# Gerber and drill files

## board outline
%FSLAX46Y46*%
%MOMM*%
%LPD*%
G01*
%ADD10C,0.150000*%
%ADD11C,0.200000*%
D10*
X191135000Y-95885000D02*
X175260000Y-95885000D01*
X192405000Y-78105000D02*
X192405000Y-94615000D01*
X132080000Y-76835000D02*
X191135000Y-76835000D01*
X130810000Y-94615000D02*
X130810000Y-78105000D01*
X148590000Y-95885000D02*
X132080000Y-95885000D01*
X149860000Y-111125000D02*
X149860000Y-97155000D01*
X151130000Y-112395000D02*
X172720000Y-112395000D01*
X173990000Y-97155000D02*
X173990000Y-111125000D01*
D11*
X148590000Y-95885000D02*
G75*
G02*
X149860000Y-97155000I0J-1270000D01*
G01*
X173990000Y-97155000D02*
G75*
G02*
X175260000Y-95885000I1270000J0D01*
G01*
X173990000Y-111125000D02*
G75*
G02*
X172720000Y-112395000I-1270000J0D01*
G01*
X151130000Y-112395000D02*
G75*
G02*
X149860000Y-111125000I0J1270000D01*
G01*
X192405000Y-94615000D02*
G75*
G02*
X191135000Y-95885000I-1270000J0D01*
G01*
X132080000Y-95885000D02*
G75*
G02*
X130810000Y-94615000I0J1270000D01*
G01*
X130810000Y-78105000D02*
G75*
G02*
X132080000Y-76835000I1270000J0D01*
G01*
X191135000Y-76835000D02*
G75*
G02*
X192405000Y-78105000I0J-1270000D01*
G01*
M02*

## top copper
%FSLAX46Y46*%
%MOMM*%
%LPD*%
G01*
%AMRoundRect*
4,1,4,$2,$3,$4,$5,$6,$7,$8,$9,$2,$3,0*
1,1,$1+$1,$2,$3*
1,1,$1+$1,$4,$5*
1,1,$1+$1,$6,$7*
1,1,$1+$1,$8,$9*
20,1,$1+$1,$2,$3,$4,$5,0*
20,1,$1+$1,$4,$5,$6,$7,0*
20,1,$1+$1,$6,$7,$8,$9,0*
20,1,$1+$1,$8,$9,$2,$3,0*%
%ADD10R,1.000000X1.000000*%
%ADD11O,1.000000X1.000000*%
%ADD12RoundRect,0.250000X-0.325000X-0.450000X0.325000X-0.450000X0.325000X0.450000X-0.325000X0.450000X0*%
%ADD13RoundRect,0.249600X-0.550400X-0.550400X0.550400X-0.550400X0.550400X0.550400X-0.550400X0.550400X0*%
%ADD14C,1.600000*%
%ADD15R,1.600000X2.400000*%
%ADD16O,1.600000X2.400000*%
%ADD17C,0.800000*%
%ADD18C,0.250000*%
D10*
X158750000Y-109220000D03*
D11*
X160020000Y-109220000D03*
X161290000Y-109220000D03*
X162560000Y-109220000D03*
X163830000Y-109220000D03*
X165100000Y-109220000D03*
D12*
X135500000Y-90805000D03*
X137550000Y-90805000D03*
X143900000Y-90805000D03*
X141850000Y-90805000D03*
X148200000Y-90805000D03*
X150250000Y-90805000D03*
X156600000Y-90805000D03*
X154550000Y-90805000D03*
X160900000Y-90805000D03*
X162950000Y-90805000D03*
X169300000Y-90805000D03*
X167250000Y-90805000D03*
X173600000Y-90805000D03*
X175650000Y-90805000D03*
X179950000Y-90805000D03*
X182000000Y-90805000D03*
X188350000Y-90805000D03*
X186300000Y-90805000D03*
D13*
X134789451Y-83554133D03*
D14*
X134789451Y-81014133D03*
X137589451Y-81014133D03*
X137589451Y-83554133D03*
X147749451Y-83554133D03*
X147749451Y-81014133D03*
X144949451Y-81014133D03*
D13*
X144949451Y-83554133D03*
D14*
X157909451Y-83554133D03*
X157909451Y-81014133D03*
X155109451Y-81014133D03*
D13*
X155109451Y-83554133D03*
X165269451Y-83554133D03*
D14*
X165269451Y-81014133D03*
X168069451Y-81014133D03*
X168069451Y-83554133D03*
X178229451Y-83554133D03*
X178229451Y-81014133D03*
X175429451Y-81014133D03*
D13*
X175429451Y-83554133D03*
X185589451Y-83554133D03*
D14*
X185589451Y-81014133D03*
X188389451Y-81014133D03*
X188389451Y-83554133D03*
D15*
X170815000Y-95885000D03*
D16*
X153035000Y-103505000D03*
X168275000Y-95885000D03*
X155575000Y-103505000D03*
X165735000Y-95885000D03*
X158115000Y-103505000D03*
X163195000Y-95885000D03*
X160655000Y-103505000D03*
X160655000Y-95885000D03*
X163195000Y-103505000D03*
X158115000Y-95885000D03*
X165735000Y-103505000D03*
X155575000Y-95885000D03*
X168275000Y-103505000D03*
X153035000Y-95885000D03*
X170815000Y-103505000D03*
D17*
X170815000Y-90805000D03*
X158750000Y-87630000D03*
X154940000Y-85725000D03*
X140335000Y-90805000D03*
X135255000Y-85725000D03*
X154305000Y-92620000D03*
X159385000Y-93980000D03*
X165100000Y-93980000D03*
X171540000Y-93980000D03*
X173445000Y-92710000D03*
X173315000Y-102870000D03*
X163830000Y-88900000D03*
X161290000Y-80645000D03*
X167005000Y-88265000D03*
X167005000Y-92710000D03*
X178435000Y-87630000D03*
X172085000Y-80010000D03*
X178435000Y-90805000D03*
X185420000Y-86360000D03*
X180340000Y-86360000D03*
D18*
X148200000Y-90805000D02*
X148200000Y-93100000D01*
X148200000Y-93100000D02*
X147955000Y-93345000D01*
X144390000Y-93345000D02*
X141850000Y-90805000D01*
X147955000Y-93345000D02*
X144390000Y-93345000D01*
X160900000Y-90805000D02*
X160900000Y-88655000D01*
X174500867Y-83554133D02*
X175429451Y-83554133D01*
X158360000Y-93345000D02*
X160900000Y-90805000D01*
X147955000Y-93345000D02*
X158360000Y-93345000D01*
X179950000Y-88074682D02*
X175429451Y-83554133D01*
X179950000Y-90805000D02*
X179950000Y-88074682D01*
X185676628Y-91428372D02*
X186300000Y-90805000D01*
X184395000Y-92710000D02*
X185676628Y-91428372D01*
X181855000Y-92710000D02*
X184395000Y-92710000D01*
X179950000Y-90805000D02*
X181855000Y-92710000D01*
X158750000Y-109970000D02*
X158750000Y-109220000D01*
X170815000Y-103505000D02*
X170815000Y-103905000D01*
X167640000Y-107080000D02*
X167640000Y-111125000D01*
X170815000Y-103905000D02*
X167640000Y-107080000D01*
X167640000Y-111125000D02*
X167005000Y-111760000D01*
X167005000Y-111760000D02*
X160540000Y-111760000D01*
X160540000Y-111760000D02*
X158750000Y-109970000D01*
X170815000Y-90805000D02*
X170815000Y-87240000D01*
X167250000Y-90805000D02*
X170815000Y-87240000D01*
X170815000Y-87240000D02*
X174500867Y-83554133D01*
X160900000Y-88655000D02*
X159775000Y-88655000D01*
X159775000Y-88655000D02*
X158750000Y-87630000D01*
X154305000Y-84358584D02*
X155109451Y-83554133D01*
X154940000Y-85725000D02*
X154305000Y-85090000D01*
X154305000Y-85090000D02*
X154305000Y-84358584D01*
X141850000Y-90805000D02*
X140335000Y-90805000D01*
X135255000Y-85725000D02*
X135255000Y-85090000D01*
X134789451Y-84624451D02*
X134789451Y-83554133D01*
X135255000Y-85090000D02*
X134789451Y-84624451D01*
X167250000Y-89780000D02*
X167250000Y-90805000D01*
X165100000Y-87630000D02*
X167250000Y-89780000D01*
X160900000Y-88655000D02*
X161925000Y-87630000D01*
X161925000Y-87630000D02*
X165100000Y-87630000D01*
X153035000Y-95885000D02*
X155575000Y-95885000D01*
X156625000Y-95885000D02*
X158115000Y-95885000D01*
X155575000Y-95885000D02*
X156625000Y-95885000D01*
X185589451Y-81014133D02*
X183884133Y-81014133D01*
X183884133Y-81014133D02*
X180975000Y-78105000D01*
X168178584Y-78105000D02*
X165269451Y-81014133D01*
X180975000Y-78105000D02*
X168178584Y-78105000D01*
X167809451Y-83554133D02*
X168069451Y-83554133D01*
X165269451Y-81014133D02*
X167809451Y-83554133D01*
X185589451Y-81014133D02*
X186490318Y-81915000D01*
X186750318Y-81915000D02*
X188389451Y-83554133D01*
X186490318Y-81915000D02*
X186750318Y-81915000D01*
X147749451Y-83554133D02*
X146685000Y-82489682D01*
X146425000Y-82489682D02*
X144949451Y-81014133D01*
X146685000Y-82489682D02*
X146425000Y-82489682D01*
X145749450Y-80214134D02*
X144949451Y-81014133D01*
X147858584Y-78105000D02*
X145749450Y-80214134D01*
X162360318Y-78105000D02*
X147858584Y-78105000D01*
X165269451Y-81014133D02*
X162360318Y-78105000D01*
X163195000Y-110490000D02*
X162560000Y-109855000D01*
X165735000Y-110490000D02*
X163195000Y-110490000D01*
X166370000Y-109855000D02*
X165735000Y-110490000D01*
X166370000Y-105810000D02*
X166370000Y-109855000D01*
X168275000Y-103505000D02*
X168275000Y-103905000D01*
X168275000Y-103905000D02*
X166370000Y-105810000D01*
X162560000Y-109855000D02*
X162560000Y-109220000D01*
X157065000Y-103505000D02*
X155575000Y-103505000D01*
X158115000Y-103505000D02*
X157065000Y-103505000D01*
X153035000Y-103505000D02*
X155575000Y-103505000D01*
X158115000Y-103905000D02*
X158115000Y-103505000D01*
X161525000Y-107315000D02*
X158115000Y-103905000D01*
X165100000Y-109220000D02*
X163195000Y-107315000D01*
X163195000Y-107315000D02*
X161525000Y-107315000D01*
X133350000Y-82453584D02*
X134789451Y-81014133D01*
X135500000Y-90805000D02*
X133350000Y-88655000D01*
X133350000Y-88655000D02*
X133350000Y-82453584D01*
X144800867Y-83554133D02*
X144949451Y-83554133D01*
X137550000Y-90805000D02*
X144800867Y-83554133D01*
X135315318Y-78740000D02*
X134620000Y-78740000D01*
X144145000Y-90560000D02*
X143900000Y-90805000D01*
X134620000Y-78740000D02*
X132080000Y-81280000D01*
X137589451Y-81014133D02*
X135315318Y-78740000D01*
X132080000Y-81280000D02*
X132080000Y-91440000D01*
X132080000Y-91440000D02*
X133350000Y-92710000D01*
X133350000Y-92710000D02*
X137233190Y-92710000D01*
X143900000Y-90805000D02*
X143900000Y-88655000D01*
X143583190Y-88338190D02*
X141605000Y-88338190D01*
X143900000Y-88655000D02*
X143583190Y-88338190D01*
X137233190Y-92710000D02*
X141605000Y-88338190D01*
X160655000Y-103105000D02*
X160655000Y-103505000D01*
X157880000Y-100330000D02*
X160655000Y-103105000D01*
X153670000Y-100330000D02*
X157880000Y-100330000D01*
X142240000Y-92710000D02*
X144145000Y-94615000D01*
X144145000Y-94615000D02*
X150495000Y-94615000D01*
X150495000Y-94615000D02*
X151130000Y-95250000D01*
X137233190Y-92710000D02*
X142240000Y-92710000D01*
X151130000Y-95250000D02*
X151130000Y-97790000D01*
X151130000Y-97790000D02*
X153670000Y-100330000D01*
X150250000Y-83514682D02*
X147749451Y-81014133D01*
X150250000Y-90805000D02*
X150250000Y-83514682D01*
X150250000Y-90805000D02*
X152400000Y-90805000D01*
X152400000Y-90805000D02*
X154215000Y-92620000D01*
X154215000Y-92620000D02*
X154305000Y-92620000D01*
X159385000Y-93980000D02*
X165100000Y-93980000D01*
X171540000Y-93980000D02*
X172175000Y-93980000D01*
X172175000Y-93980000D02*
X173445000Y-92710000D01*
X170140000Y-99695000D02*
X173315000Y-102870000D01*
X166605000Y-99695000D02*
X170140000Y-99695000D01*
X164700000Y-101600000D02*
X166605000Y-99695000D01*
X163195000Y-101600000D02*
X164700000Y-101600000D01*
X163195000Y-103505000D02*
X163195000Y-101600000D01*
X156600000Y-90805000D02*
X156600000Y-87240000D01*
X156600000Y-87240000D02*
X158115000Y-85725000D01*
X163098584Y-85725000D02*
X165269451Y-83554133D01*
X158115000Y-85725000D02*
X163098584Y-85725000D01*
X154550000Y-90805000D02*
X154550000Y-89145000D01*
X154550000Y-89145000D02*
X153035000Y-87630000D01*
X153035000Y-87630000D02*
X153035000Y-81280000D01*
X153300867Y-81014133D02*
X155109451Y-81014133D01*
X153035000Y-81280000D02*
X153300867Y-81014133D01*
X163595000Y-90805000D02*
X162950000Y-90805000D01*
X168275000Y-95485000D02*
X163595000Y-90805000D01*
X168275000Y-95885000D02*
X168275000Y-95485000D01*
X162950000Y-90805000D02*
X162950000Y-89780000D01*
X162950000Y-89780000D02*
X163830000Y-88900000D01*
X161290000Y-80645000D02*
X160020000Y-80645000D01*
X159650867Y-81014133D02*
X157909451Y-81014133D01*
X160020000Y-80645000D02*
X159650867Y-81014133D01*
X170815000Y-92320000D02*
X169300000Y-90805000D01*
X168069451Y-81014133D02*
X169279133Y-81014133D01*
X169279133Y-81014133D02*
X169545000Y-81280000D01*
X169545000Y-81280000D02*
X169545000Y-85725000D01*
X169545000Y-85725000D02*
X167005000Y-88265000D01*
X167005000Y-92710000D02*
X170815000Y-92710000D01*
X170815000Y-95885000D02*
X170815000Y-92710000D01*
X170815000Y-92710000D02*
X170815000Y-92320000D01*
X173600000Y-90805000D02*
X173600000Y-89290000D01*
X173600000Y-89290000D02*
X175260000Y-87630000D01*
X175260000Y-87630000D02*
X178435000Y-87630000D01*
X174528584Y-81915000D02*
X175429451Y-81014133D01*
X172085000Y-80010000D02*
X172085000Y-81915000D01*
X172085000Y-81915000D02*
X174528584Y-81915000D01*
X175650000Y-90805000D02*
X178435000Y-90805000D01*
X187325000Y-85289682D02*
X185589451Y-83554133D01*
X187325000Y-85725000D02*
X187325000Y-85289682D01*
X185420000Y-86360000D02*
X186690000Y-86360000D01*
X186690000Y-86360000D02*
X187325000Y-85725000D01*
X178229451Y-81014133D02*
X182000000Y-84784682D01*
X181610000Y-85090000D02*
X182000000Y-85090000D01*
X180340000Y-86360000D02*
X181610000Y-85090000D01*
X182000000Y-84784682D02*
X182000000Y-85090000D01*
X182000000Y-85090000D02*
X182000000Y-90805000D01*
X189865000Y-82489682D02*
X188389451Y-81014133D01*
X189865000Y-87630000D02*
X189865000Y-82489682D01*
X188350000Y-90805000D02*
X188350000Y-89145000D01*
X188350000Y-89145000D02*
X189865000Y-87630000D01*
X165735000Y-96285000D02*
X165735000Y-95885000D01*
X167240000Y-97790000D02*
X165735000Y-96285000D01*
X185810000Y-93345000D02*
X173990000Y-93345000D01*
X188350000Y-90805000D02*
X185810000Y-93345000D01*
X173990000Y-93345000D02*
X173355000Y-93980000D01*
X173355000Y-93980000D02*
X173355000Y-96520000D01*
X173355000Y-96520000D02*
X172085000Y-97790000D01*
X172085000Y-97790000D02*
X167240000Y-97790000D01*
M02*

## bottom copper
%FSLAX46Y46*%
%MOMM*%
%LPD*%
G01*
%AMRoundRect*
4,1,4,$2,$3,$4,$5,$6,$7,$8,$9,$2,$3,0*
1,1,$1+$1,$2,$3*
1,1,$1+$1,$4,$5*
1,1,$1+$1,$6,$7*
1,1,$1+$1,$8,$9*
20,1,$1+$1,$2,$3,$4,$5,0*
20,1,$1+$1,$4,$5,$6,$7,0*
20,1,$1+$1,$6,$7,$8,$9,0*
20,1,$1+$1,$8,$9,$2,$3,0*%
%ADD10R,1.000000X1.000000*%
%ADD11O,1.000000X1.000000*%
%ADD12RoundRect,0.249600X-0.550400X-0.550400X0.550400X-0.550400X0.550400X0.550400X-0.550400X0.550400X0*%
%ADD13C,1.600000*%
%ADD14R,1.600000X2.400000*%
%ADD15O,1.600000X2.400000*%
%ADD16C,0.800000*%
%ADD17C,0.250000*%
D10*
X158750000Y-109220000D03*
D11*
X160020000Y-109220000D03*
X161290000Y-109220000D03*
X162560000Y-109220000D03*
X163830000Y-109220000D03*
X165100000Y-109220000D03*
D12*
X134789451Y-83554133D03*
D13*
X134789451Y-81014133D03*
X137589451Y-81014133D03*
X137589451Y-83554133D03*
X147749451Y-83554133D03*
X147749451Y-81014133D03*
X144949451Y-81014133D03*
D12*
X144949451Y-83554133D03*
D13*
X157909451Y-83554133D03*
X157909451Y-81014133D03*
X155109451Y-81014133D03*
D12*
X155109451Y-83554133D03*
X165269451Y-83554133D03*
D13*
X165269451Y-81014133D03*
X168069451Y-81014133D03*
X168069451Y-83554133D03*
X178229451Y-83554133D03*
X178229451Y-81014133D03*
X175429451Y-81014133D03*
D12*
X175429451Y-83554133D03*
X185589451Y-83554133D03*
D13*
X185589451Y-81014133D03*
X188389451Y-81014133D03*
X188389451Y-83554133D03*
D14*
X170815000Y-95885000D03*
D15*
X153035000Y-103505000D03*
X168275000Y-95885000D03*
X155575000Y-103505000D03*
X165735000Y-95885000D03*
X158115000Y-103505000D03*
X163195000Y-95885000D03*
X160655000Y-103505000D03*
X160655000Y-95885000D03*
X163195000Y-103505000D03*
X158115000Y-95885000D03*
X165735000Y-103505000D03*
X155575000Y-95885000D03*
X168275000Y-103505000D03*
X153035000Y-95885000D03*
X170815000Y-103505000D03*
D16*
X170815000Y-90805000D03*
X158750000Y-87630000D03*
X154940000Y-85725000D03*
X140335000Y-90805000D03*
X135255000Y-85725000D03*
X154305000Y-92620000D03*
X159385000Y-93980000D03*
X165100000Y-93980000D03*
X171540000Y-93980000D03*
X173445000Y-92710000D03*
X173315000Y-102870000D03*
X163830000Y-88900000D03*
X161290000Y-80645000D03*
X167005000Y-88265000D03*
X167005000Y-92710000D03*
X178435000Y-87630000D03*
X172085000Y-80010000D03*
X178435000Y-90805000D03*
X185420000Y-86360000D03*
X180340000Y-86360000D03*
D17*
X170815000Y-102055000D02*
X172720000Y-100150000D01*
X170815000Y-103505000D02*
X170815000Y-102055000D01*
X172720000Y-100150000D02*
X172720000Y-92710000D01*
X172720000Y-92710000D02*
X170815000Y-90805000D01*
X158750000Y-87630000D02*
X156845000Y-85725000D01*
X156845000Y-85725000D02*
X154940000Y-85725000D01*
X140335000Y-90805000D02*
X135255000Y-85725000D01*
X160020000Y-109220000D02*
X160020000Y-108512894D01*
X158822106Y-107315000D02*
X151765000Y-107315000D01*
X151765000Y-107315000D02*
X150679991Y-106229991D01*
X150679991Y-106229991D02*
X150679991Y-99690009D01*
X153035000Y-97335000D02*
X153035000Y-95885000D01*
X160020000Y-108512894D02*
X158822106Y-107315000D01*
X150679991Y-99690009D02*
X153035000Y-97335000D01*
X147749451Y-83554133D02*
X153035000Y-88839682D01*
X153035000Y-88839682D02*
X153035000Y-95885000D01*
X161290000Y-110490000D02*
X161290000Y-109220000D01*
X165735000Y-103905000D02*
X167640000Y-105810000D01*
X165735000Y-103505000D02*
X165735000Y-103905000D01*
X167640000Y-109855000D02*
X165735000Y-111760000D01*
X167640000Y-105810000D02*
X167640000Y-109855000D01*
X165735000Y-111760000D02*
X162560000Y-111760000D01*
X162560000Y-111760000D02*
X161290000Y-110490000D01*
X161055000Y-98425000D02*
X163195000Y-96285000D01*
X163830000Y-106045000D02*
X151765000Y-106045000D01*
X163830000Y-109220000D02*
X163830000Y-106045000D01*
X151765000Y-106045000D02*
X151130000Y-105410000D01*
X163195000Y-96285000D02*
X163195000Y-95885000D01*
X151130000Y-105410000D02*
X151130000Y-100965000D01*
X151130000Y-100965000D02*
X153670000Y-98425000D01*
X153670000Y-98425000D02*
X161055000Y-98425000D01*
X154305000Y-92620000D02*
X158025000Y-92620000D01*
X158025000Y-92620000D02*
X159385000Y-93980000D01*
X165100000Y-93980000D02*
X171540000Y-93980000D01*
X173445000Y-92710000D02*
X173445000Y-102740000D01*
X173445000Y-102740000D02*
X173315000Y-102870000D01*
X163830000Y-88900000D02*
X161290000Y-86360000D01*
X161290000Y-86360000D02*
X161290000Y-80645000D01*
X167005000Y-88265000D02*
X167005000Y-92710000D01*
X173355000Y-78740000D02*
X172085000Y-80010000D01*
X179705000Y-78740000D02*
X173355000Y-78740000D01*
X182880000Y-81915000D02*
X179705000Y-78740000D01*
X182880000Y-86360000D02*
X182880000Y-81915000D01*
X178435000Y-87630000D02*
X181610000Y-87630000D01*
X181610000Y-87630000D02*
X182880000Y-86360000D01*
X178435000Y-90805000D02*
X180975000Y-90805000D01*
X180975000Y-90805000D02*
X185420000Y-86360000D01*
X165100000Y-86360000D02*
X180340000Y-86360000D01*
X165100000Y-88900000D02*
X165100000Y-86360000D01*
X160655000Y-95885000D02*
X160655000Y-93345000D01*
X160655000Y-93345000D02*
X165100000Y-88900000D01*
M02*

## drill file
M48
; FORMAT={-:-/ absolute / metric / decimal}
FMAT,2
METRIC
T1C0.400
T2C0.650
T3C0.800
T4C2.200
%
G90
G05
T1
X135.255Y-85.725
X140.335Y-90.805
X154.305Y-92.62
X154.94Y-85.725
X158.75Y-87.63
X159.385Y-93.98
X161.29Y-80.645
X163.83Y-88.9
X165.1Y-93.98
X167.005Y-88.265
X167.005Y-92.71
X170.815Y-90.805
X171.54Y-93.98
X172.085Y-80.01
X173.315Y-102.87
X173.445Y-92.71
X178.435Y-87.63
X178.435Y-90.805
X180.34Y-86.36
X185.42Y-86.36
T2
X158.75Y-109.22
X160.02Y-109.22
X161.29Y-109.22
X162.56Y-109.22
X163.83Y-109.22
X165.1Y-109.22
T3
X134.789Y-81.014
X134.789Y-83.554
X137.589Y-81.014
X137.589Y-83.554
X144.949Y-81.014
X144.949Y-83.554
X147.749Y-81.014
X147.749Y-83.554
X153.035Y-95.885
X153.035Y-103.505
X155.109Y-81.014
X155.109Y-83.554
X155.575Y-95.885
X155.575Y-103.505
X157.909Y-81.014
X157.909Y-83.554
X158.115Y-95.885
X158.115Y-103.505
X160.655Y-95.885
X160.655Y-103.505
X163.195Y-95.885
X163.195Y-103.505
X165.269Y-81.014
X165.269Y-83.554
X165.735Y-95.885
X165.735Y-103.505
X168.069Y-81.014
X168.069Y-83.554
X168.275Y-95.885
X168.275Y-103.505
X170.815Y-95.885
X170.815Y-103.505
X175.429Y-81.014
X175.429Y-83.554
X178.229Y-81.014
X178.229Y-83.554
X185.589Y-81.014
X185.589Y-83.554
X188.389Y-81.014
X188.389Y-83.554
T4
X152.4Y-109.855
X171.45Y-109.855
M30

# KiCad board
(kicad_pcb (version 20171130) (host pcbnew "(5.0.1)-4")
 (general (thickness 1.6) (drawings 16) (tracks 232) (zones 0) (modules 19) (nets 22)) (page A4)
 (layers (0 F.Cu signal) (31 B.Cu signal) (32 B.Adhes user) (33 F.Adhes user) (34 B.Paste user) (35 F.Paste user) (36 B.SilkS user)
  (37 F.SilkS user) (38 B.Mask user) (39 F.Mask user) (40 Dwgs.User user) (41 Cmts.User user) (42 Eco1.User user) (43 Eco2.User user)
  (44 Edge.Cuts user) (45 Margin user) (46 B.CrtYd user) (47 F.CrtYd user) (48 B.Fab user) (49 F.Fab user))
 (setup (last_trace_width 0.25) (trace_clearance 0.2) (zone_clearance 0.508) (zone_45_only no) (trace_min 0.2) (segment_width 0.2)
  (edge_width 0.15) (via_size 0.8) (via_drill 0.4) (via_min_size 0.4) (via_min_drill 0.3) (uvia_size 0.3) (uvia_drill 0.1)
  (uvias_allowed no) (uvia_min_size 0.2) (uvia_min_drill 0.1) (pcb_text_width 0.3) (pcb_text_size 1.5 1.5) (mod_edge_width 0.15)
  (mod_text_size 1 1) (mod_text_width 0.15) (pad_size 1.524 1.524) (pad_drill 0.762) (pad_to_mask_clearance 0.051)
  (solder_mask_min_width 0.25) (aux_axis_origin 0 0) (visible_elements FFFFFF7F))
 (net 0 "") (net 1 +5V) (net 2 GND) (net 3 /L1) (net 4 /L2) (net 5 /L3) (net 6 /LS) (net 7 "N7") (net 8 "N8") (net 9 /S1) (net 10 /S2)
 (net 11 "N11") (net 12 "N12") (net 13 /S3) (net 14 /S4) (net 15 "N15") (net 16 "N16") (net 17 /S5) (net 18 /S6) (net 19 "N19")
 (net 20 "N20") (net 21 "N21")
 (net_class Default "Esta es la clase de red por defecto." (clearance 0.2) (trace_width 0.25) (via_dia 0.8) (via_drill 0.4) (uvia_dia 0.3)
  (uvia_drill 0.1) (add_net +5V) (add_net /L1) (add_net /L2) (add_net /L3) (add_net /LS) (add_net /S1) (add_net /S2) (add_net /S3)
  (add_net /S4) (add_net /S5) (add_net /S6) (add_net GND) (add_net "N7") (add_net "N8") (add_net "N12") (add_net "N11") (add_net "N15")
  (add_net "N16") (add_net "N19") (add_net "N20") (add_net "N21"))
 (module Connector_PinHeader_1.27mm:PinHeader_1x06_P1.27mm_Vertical (layer F.Cu) (at 158.75 109.22 90)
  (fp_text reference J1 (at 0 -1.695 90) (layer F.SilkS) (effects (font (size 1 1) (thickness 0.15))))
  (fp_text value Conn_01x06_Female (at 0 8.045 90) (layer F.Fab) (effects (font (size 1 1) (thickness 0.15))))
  (pad 1 thru_hole rect (at 0 0 90) (size 1 1) (drill 0.65) (layers *.Cu *.Mask) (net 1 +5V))
  (pad 2 thru_hole oval (at 0 1.27 90) (size 1 1) (drill 0.65) (layers *.Cu *.Mask) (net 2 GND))
  (pad 3 thru_hole oval (at 0 2.54 90) (size 1 1) (drill 0.65) (layers *.Cu *.Mask) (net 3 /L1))
  (pad 4 thru_hole oval (at 0 3.81 90) (size 1 1) (drill 0.65) (layers *.Cu *.Mask) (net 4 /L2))
  (pad 5 thru_hole oval (at 0 5.08 90) (size 1 1) (drill 0.65) (layers *.Cu *.Mask) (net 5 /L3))
  (pad 6 thru_hole oval (at 0 6.35 90) (size 1 1) (drill 0.65) (layers *.Cu *.Mask) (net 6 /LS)))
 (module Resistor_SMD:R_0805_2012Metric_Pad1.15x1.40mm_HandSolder (layer F.Cu) (at 136.525 90.805)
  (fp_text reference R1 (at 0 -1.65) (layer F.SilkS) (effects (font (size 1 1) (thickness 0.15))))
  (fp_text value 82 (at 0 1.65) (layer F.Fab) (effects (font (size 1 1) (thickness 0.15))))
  (pad 1 smd roundrect (at -1.025 0) (size 1.15 1.4) (layers F.Cu F.Paste F.Mask) (roundrect_rratio 0.217391) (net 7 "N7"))
  (pad 2 smd roundrect (at 1.025 0) (size 1.15 1.4) (layers F.Cu F.Paste F.Mask) (roundrect_rratio 0.217391) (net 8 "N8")))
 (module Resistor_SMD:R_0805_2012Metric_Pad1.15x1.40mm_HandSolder (layer F.Cu) (at 142.875 90.805)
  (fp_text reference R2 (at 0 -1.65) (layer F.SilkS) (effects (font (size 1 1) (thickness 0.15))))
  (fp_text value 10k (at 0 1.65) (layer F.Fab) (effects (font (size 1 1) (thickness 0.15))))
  (pad 2 smd roundrect (at 1.025 0) (size 1.15 1.4) (layers F.Cu F.Paste F.Mask) (roundrect_rratio 0.217391) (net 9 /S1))
  (pad 1 smd roundrect (at -1.025 0) (size 1.15 1.4) (layers F.Cu F.Paste F.Mask) (roundrect_rratio 0.217391) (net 1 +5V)))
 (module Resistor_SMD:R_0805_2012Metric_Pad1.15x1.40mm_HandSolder (layer F.Cu) (at 149.225 90.805)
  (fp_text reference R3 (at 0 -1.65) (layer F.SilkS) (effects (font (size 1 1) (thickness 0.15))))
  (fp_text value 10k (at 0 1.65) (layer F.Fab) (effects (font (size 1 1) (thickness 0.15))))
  (pad 1 smd roundrect (at -1.025 0) (size 1.15 1.4) (layers F.Cu F.Paste F.Mask) (roundrect_rratio 0.217391) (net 1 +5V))
  (pad 2 smd roundrect (at 1.025 0) (size 1.15 1.4) (layers F.Cu F.Paste F.Mask) (roundrect_rratio 0.217391) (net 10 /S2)))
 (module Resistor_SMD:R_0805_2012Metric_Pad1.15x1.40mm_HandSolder (layer F.Cu) (at 155.575 90.805)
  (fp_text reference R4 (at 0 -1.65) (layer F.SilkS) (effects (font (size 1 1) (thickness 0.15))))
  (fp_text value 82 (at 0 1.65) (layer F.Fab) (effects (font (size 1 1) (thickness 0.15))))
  (pad 2 smd roundrect (at 1.025 0) (size 1.15 1.4) (layers F.Cu F.Paste F.Mask) (roundrect_rratio 0.217391) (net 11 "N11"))
  (pad 1 smd roundrect (at -1.025 0) (size 1.15 1.4) (layers F.Cu F.Paste F.Mask) (roundrect_rratio 0.217391) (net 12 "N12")))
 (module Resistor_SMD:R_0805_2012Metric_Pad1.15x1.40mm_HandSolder (layer F.Cu) (at 161.925 90.805)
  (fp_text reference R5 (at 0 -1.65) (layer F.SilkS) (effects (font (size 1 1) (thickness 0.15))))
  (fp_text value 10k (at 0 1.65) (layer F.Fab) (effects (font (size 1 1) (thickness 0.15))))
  (pad 1 smd roundrect (at -1.025 0) (size 1.15 1.4) (layers F.Cu F.Paste F.Mask) (roundrect_rratio 0.217391) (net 1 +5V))
  (pad 2 smd roundrect (at 1.025 0) (size 1.15 1.4) (layers F.Cu F.Paste F.Mask) (roundrect_rratio 0.217391) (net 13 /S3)))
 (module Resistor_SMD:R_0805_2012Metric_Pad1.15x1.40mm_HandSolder (layer F.Cu) (at 168.275 90.805)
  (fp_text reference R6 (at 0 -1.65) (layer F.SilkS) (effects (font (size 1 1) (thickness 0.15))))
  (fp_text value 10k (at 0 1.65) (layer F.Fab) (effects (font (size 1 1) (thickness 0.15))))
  (pad 2 smd roundrect (at 1.025 0) (size 1.15 1.4) (layers F.Cu F.Paste F.Mask) (roundrect_rratio 0.217391) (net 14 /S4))
  (pad 1 smd roundrect (at -1.025 0) (size 1.15 1.4) (layers F.Cu F.Paste F.Mask) (roundrect_rratio 0.217391) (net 1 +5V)))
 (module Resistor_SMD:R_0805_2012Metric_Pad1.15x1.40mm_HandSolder (layer F.Cu) (at 174.625 90.805)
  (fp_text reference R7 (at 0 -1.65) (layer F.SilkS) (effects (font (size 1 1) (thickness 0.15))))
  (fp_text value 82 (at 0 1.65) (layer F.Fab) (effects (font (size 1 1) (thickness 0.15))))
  (pad 1 smd roundrect (at -1.025 0) (size 1.15 1.4) (layers F.Cu F.Paste F.Mask) (roundrect_rratio 0.217391) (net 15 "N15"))
  (pad 2 smd roundrect (at 1.025 0) (size 1.15 1.4) (layers F.Cu F.Paste F.Mask) (roundrect_rratio 0.217391) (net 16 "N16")))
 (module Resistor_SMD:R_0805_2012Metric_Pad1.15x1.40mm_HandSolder (layer F.Cu) (at 180.975 90.805)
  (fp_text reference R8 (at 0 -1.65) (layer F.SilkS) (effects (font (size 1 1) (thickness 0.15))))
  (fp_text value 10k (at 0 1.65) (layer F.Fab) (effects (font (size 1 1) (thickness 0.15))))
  (pad 1 smd roundrect (at -1.025 0) (size 1.15 1.4) (layers F.Cu F.Paste F.Mask) (roundrect_rratio 0.217391) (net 1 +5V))
  (pad 2 smd roundrect (at 1.025 0) (size 1.15 1.4) (layers F.Cu F.Paste F.Mask) (roundrect_rratio 0.217391) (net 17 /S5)))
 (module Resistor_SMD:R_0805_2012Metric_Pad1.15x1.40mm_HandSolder (layer F.Cu) (at 187.325 90.805)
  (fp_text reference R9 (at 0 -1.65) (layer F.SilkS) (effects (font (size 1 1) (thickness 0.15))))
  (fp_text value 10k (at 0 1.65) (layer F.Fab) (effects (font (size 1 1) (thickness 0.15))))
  (pad 2 smd roundrect (at 1.025 0) (size 1.15 1.4) (layers F.Cu F.Paste F.Mask) (roundrect_rratio 0.217391) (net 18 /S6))
  (pad 1 smd roundrect (at -1.025 0) (size 1.15 1.4) (layers F.Cu F.Paste F.Mask) (roundrect_rratio 0.217391) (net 1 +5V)))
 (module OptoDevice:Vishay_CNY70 (layer B.Cu) (at 134.789451 83.554133)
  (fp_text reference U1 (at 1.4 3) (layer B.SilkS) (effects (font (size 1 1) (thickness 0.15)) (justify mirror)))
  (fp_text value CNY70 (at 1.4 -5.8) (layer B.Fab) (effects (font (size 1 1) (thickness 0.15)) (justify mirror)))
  (pad 1 thru_hole roundrect (at 0 0) (size 1.6 1.6) (drill 0.8) (layers *.Cu *.Mask) (roundrect_rratio 0.156) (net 1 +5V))
  (pad 2 thru_hole circle (at 0 -2.54) (size 1.6 1.6) (drill 0.8) (layers *.Cu *.Mask) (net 7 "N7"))
  (pad 3 thru_hole circle (at 2.8 -2.54) (size 1.6 1.6) (drill 0.8) (layers *.Cu *.Mask) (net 9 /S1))
  (pad 4 thru_hole circle (at 2.8 0) (size 1.6 1.6) (drill 0.8) (layers *.Cu *.Mask) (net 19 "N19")))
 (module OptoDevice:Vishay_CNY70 (layer B.Cu) (at 144.949451 83.554133)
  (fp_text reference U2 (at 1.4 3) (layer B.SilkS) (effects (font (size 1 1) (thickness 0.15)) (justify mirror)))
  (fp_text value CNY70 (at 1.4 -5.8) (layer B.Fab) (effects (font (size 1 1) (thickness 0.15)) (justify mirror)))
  (pad 4 thru_hole circle (at 2.8 0) (size 1.6 1.6) (drill 0.8) (layers *.Cu *.Mask) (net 2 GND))
  (pad 3 thru_hole circle (at 2.8 -2.54) (size 1.6 1.6) (drill 0.8) (layers *.Cu *.Mask) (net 10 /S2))
  (pad 2 thru_hole circle (at 0 -2.54) (size 1.6 1.6) (drill 0.8) (layers *.Cu *.Mask) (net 2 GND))
  (pad 1 thru_hole roundrect (at 0 0) (size 1.6 1.6) (drill 0.8) (layers *.Cu *.Mask) (roundrect_rratio 0.156) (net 8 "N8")))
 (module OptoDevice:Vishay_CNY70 (layer B.Cu) (at 155.109451 83.554133)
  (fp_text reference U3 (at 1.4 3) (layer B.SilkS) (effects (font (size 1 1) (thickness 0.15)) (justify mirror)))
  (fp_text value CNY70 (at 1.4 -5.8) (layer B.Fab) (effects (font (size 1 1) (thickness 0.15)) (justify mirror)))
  (pad 4 thru_hole circle (at 2.8 0) (size 1.6 1.6) (drill 0.8) (layers *.Cu *.Mask) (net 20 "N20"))
  (pad 3 thru_hole circle (at 2.8 -2.54) (size 1.6 1.6) (drill 0.8) (layers *.Cu *.Mask) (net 13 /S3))
  (pad 2 thru_hole circle (at 0 -2.54) (size 1.6 1.6) (drill 0.8) (layers *.Cu *.Mask) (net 12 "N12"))
  (pad 1 thru_hole roundrect (at 0 0) (size 1.6 1.6) (drill 0.8) (layers *.Cu *.Mask) (roundrect_rratio 0.156) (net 1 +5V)))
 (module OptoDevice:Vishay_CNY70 (layer B.Cu) (at 165.269451 83.554133)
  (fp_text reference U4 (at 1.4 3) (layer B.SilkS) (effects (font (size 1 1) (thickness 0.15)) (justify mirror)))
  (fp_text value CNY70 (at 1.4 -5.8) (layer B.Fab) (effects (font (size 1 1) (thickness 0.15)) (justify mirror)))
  (pad 1 thru_hole roundrect (at 0 0) (size 1.6 1.6) (drill 0.8) (layers *.Cu *.Mask) (roundrect_rratio 0.156) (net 11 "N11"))
  (pad 2 thru_hole circle (at 0 -2.54) (size 1.6 1.6) (drill 0.8) (layers *.Cu *.Mask) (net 2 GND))
  (pad 3 thru_hole circle (at 2.8 -2.54) (size 1.6 1.6) (drill 0.8) (layers *.Cu *.Mask) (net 14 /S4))
  (pad 4 thru_hole circle (at 2.8 0) (size 1.6 1.6) (drill 0.8) (layers *.Cu *.Mask) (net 2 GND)))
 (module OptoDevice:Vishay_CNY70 (layer B.Cu) (at 175.429451 83.554133)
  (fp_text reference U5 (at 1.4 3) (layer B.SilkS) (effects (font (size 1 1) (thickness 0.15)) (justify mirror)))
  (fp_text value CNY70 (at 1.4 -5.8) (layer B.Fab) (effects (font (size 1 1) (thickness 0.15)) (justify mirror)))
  (pad 4 thru_hole circle (at 2.8 0) (size 1.6 1.6) (drill 0.8) (layers *.Cu *.Mask) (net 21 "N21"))
  (pad 3 thru_hole circle (at 2.8 -2.54) (size 1.6 1.6) (drill 0.8) (layers *.Cu *.Mask) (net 17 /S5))
  (pad 2 thru_hole circle (at 0 -2.54) (size 1.6 1.6) (drill 0.8) (layers *.Cu *.Mask) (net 15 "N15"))
  (pad 1 thru_hole roundrect (at 0 0) (size 1.6 1.6) (drill 0.8) (layers *.Cu *.Mask) (roundrect_rratio 0.156) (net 1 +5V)))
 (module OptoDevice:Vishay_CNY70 (layer B.Cu) (at 185.589451 83.554133)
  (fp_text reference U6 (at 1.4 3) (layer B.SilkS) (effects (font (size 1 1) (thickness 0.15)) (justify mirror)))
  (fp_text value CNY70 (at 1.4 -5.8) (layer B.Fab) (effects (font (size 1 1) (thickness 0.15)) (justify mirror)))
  (pad 1 thru_hole roundrect (at 0 0) (size 1.6 1.6) (drill 0.8) (layers *.Cu *.Mask) (roundrect_rratio 0.156) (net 16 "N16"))
  (pad 2 thru_hole circle (at 0 -2.54) (size 1.6 1.6) (drill 0.8) (layers *.Cu *.Mask) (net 2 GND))
  (pad 3 thru_hole circle (at 2.8 -2.54) (size 1.6 1.6) (drill 0.8) (layers *.Cu *.Mask) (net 18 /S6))
  (pad 4 thru_hole circle (at 2.8 0) (size 1.6 1.6) (drill 0.8) (layers *.Cu *.Mask) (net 2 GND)))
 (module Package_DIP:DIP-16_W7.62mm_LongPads (layer F.Cu) (at 170.815 95.885 270)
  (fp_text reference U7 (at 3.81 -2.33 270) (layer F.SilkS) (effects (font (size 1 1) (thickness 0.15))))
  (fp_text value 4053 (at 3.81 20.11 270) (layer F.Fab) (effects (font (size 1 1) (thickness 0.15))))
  (pad 1 thru_hole rect (at 0 0 270) (size 2.4 1.6) (drill 0.8) (layers *.Cu *.Mask) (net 14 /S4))
  (pad 9 thru_hole oval (at 7.62 17.78 270) (size 2.4 1.6) (drill 0.8) (layers *.Cu *.Mask) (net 6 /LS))
  (pad 2 thru_hole oval (at 0 2.54 270) (size 2.4 1.6) (drill 0.8) (layers *.Cu *.Mask) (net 13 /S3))
  (pad 10 thru_hole oval (at 7.62 15.24 270) (size 2.4 1.6) (drill 0.8) (layers *.Cu *.Mask) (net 6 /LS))
  (pad 3 thru_hole oval (at 0 5.08 270) (size 2.4 1.6) (drill 0.8) (layers *.Cu *.Mask) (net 18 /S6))
  (pad 11 thru_hole oval (at 7.62 12.7 270) (size 2.4 1.6) (drill 0.8) (layers *.Cu *.Mask) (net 6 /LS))
  (pad 4 thru_hole oval (at 0 7.62 270) (size 2.4 1.6) (drill 0.8) (layers *.Cu *.Mask) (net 5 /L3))
  (pad 12 thru_hole oval (at 7.62 10.16 270) (size 2.4 1.6) (drill 0.8) (layers *.Cu *.Mask) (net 9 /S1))
  (pad 5 thru_hole oval (at 0 10.16 270) (size 2.4 1.6) (drill 0.8) (layers *.Cu *.Mask) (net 17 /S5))
  (pad 13 thru_hole oval (at 7.62 7.62 270) (size 2.4 1.6) (drill 0.8) (layers *.Cu *.Mask) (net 10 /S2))
  (pad 6 thru_hole oval (at 0 12.7 270) (size 2.4 1.6) (drill 0.8) (layers *.Cu *.Mask) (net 2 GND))
  (pad 14 thru_hole oval (at 7.62 5.08 270) (size 2.4 1.6) (drill 0.8) (layers *.Cu *.Mask) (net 3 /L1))
  (pad 7 thru_hole oval (at 0 15.24 270) (size 2.4 1.6) (drill 0.8) (layers *.Cu *.Mask) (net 2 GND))
  (pad 15 thru_hole oval (at 7.62 2.54 270) (size 2.4 1.6) (drill 0.8) (layers *.Cu *.Mask) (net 4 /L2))
  (pad 8 thru_hole oval (at 0 17.78 270) (size 2.4 1.6) (drill 0.8) (layers *.Cu *.Mask) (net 2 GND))
  (pad 16 thru_hole oval (at 7.62 0 270) (size 2.4 1.6) (drill 0.8) (layers *.Cu *.Mask) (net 1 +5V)))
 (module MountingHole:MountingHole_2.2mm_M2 (layer F.Cu) (at 152.4 109.855)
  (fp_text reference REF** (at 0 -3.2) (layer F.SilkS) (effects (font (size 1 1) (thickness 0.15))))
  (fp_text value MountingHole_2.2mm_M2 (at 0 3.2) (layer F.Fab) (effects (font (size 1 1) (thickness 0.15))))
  (pad 1 np_thru_hole circle (at 0 0) (size 2.2 2.2) (drill 2.2) (layers *.Cu *.Mask)))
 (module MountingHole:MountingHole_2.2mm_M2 (layer F.Cu) (at 171.45 109.855)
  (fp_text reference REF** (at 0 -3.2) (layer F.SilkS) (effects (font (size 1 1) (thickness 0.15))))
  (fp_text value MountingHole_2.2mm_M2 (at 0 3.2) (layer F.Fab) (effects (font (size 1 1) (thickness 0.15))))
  (pad 1 np_thru_hole circle (at 0 0) (size 2.2 2.2) (drill 2.2) (layers *.Cu *.Mask)))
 (gr_line (start 191.135 95.885) (end 175.26 95.885) (layer Edge.Cuts) (width 0.15))
 (gr_line (start 192.405 78.105) (end 192.405 94.615) (layer Edge.Cuts) (width 0.15))
 (gr_line (start 132.08 76.835) (end 191.135 76.835) (layer Edge.Cuts) (width 0.15))
 (gr_line (start 130.81 94.615) (end 130.81 78.105) (layer Edge.Cuts) (width 0.15))
 (gr_line (start 148.59 95.885) (end 132.08 95.885) (layer Edge.Cuts) (width 0.15))
 (gr_line (start 149.86 111.125) (end 149.86 97.155) (layer Edge.Cuts) (width 0.15))
 (gr_line (start 151.13 112.395) (end 172.72 112.395) (layer Edge.Cuts) (width 0.15))
 (gr_line (start 173.99 97.155) (end 173.99 111.125) (layer Edge.Cuts) (width 0.15))
 (gr_arc (start 148.59 97.155) (end 149.86 97.155) (angle -90) (layer Edge.Cuts) (width 0.2))
 (gr_arc (start 175.26 97.155) (end 175.26 95.885) (angle -90) (layer Edge.Cuts) (width 0.2))
 (gr_arc (start 172.72 111.125) (end 172.72 112.395) (angle -90) (layer Edge.Cuts) (width 0.2))
 (gr_arc (start 151.13 111.125) (end 149.86 111.125) (angle -90) (layer Edge.Cuts) (width 0.2))
 (gr_arc (start 191.135 94.615) (end 191.135 95.885) (angle -90) (layer Edge.Cuts) (width 0.2))
 (gr_arc (start 132.08 94.615) (end 130.81 94.615) (angle -90) (layer Edge.Cuts) (width 0.2))
 (gr_arc (start 132.08 78.105) (end 132.08 76.835) (angle -90) (layer Edge.Cuts) (width 0.2))
 (gr_arc (start 191.135 78.105) (end 192.405 78.105) (angle -90) (layer Edge.Cuts) (width 0.2))
 (segment (start 148.2 90.805) (end 148.2 93.1) (width 0.25) (layer F.Cu) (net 1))
 (segment (start 148.2 93.1) (end 147.955 93.345) (width 0.25) (layer F.Cu) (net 1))
 (segment (start 144.39 93.345) (end 141.85 90.805) (width 0.25) (layer F.Cu) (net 1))
 (segment (start 147.955 93.345) (end 144.39 93.345) (width 0.25) (layer F.Cu) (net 1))
 (segment (start 160.9 90.805) (end 160.9 88.655) (width 0.25) (layer F.Cu) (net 1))
 (segment (start 174.500867 83.554133) (end 175.429451 83.554133) (width 0.25) (layer F.Cu) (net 1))
 (segment (start 158.36 93.345) (end 160.9 90.805) (width 0.25) (layer F.Cu) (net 1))
 (segment (start 147.955 93.345) (end 158.36 93.345) (width 0.25) (layer F.Cu) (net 1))
 (segment (start 179.95 88.074682) (end 175.429451 83.554133) (width 0.25) (layer F.Cu) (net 1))
 (segment (start 179.95 90.805) (end 179.95 88.074682) (width 0.25) (layer F.Cu) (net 1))
 (segment (start 185.676628 91.428372) (end 186.3 90.805) (width 0.25) (layer F.Cu) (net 1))
 (segment (start 184.395 92.71) (end 185.676628 91.428372) (width 0.25) (layer F.Cu) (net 1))
 (segment (start 181.855 92.71) (end 184.395 92.71) (width 0.25) (layer F.Cu) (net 1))
 (segment (start 179.95 90.805) (end 181.855 92.71) (width 0.25) (layer F.Cu) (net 1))
 (segment (start 158.75 109.97) (end 158.75 109.22) (width 0.25) (layer F.Cu) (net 1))
 (segment (start 170.815 103.505) (end 170.815 103.905) (width 0.25) (layer F.Cu) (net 1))
 (segment (start 167.64 107.08) (end 167.64 111.125) (width 0.25) (layer F.Cu) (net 1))
 (segment (start 170.815 103.905) (end 167.64 107.08) (width 0.25) (layer F.Cu) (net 1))
 (segment (start 167.64 111.125) (end 167.005 111.76) (width 0.25) (layer F.Cu) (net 1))
 (segment (start 167.005 111.76) (end 160.54 111.76) (width 0.25) (layer F.Cu) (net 1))
 (segment (start 160.54 111.76) (end 158.75 109.97) (width 0.25) (layer F.Cu) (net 1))
 (segment (start 170.815 102.055) (end 172.72 100.15) (width 0.25) (layer B.Cu) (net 1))
 (segment (start 170.815 103.505) (end 170.815 102.055) (width 0.25) (layer B.Cu) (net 1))
 (via (at 170.815 90.805) (size 0.8) (drill 0.4) (layers F.Cu B.Cu) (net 1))
 (segment (start 172.72 100.15) (end 172.72 92.71) (width 0.25) (layer B.Cu) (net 1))
 (segment (start 172.72 92.71) (end 170.815 90.805) (width 0.25) (layer B.Cu) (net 1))
 (segment (start 170.815 90.805) (end 170.815 87.24) (width 0.25) (layer F.Cu) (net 1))
 (segment (start 167.25 90.805) (end 170.815 87.24) (width 0.25) (layer F.Cu) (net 1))
 (segment (start 170.815 87.24) (end 174.500867 83.554133) (width 0.25) (layer F.Cu) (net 1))
 (via (at 158.75 87.63) (size 0.8) (drill 0.4) (layers F.Cu B.Cu) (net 1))
 (segment (start 160.9 88.655) (end 159.775 88.655) (width 0.25) (layer F.Cu) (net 1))
 (segment (start 159.775 88.655) (end 158.75 87.63) (width 0.25) (layer F.Cu) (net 1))
 (via (at 154.94 85.725) (size 0.8) (drill 0.4) (layers F.Cu B.Cu) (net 1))
 (segment (start 158.75 87.63) (end 156.845 85.725) (width 0.25) (layer B.Cu) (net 1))
 (segment (start 156.845 85.725) (end 154.94 85.725) (width 0.25) (layer B.Cu) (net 1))
 (segment (start 154.305 84.358584) (end 155.109451 83.554133) (width 0.25) (layer F.Cu) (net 1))
 (segment (start 154.94 85.725) (end 154.305 85.09) (width 0.25) (layer F.Cu) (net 1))
 (segment (start 154.305 85.09) (end 154.305 84.358584) (width 0.25) (layer F.Cu) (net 1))
 (via (at 140.335 90.805) (size 0.8) (drill 0.4) (layers F.Cu B.Cu) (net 1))
 (segment (start 141.85 90.805) (end 140.335 90.805) (width 0.25) (layer F.Cu) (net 1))
 (segment (start 140.335 90.805) (end 135.255 85.725) (width 0.25) (layer B.Cu) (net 1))
 (via (at 135.255 85.725) (size 0.8) (drill 0.4) (layers F.Cu B.Cu) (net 1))
 (segment (start 135.255 85.725) (end 135.255 85.09) (width 0.25) (layer F.Cu) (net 1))
 (segment (start 134.789451 84.624451) (end 134.789451 83.554133) (width 0.25) (layer F.Cu) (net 1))
 (segment (start 135.255 85.09) (end 134.789451 84.624451) (width 0.25) (layer F.Cu) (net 1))
 (segment (start 167.25 89.78) (end 167.25 90.805) (width 0.25) (layer F.Cu) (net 1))
 (segment (start 165.1 87.63) (end 167.25 89.78) (width 0.25) (layer F.Cu) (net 1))
 (segment (start 160.9 88.655) (end 161.925 87.63) (width 0.25) (layer F.Cu) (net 1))
 (segment (start 161.925 87.63) (end 165.1 87.63) (width 0.25) (layer F.Cu) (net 1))
 (segment (start 153.035 95.885) (end 155.575 95.885) (width 0.25) (layer F.Cu) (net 2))
 (segment (start 156.625 95.885) (end 158.115 95.885) (width 0.25) (layer F.Cu) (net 2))
 (segment (start 155.575 95.885) (end 156.625 95.885) (width 0.25) (layer F.Cu) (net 2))
 (segment (start 185.589451 81.014133) (end 183.884133 81.014133) (width 0.25) (layer F.Cu) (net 2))
 (segment (start 183.884133 81.014133) (end 180.975 78.105) (width 0.25) (layer F.Cu) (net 2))
 (segment (start 168.178584 78.105) (end 165.269451 81.014133) (width 0.25) (layer F.Cu) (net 2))
 (segment (start 180.975 78.105) (end 168.178584 78.105) (width 0.25) (layer F.Cu) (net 2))
 (segment (start 167.809451 83.554133) (end 168.069451 83.554133) (width 0.25) (layer F.Cu) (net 2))
 (segment (start 165.269451 81.014133) (end 167.809451 83.554133) (width 0.25) (layer F.Cu) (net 2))
 (segment (start 185.589451 81.014133) (end 186.490318 81.915) (width 0.25) (layer F.Cu) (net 2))
 (segment (start 186.750318 81.915) (end 188.389451 83.554133) (width 0.25) (layer F.Cu) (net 2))
 (segment (start 186.490318 81.915) (end 186.750318 81.915) (width 0.25) (layer F.Cu) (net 2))
 (segment (start 147.749451 83.554133) (end 146.685 82.489682) (width 0.25) (layer F.Cu) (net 2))
 (segment (start 146.425 82.489682) (end 144.949451 81.014133) (width 0.25) (layer F.Cu) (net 2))
 (segment (start 146.685 82.489682) (end 146.425 82.489682) (width 0.25) (layer F.Cu) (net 2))
 (segment (start 145.74945 80.214134) (end 144.949451 81.014133) (width 0.25) (layer F.Cu) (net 2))
 (segment (start 147.858584 78.105) (end 145.74945 80.214134) (width 0.25) (layer F.Cu) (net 2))
 (segment (start 162.360318 78.105) (end 147.858584 78.105) (width 0.25) (layer F.Cu) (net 2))
 (segment (start 165.269451 81.014133) (end 162.360318 78.105) (width 0.25) (layer F.Cu) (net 2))
 (segment (start 160.02 109.22) (end 160.02 108.512894) (width 0.25) (layer B.Cu) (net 2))
 (segment (start 158.822106 107.315) (end 151.765 107.315) (width 0.25) (layer B.Cu) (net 2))
 (segment (start 151.765 107.315) (end 150.679991 106.229991) (width 0.25) (layer B.Cu) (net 2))
 (segment (start 150.679991 106.229991) (end 150.679991 99.690009) (width 0.25) (layer B.Cu) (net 2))
 (segment (start 153.035 97.335) (end 153.035 95.885) (width 0.25) (layer B.Cu) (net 2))
 (segment (start 160.02 108.512894) (end 158.822106 107.315) (width 0.25) (layer B.Cu) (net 2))
 (segment (start 150.679991 99.690009) (end 153.035 97.335) (width 0.25) (layer B.Cu) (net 2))
 (segment (start 147.749451 83.554133) (end 153.035 88.839682) (width 0.25) (layer B.Cu) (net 2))
 (segment (start 153.035 88.839682) (end 153.035 95.885) (width 0.25) (layer B.Cu) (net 2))
 (segment (start 161.29 110.49) (end 161.29 109.22) (width 0.25) (layer B.Cu) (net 3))
 (segment (start 165.735 103.905) (end 167.64 105.81) (width 0.25) (layer B.Cu) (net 3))
 (segment (start 165.735 103.505) (end 165.735 103.905) (width 0.25) (layer B.Cu) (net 3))
 (segment (start 167.64 109.855) (end 165.735 111.76) (width 0.25) (layer B.Cu) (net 3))
 (segment (start 167.64 105.81) (end 167.64 109.855) (width 0.25) (layer B.Cu) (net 3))
 (segment (start 165.735 111.76) (end 162.56 111.76) (width 0.25) (layer B.Cu) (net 3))
 (segment (start 162.56 111.76) (end 161.29 110.49) (width 0.25) (layer B.Cu) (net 3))
 (segment (start 163.195 110.49) (end 162.56 109.855) (width 0.25) (layer F.Cu) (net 4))
 (segment (start 165.735 110.49) (end 163.195 110.49) (width 0.25) (layer F.Cu) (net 4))
 (segment (start 166.37 109.855) (end 165.735 110.49) (width 0.25) (layer F.Cu) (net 4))
 (segment (start 166.37 105.81) (end 166.37 109.855) (width 0.25) (layer F.Cu) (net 4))
 (segment (start 168.275 103.505) (end 168.275 103.905) (width 0.25) (layer F.Cu) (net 4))
 (segment (start 168.275 103.905) (end 166.37 105.81) (width 0.25) (layer F.Cu) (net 4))
 (segment (start 162.56 109.855) (end 162.56 109.22) (width 0.25) (layer F.Cu) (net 4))
 (segment (start 161.055 98.425) (end 163.195 96.285) (width 0.25) (layer B.Cu) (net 5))
 (segment (start 163.83 106.045) (end 151.765 106.045) (width 0.25) (layer B.Cu) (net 5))
 (segment (start 163.83 109.22) (end 163.83 106.045) (width 0.25) (layer B.Cu) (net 5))
 (segment (start 151.765 106.045) (end 151.13 105.41) (width 0.25) (layer B.Cu) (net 5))
 (segment (start 163.195 96.285) (end 163.195 95.885) (width 0.25) (layer B.Cu) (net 5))
 (segment (start 151.13 105.41) (end 151.13 100.965) (width 0.25) (layer B.Cu) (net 5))
 (segment (start 151.13 100.965) (end 153.67 98.425) (width 0.25) (layer B.Cu) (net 5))
 (segment (start 153.67 98.425) (end 161.055 98.425) (width 0.25) (layer B.Cu) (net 5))
 (segment (start 157.065 103.505) (end 155.575 103.505) (width 0.25) (layer F.Cu) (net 6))
 (segment (start 158.115 103.505) (end 157.065 103.505) (width 0.25) (layer F.Cu) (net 6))
 (segment (start 153.035 103.505) (end 155.575 103.505) (width 0.25) (layer F.Cu) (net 6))
 (segment (start 158.115 103.905) (end 158.115 103.505) (width 0.25) (layer F.Cu) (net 6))
 (segment (start 161.525 107.315) (end 158.115 103.905) (width 0.25) (layer F.Cu) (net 6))
 (segment (start 165.1 109.22) (end 163.195 107.315) (width 0.25) (layer F.Cu) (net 6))
 (segment (start 163.195 107.315) (end 161.525 107.315) (width 0.25) (layer F.Cu) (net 6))
 (segment (start 133.35 82.453584) (end 134.789451 81.014133) (width 0.25) (layer F.Cu) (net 7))
 (segment (start 135.5 90.805) (end 133.35 88.655) (width 0.25) (layer F.Cu) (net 7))
 (segment (start 133.35 88.655) (end 133.35 82.453584) (width 0.25) (layer F.Cu) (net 7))
 (segment (start 144.800867 83.554133) (end 144.949451 83.554133) (width 0.25) (layer F.Cu) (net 8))
 (segment (start 137.55 90.805) (end 144.800867 83.554133) (width 0.25) (layer F.Cu) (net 8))
 (segment (start 135.315318 78.74) (end 134.62 78.74) (width 0.25) (layer F.Cu) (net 9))
 (segment (start 144.145 90.56) (end 143.9 90.805) (width 0.25) (layer F.Cu) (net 9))
 (segment (start 134.62 78.74) (end 132.08 81.28) (width 0.25) (layer F.Cu) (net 9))
 (segment (start 137.589451 81.014133) (end 135.315318 78.74) (width 0.25) (layer F.Cu) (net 9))
 (segment (start 132.08 81.28) (end 132.08 91.44) (width 0.25) (layer F.Cu) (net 9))
 (segment (start 132.08 91.44) (end 133.35 92.71) (width 0.25) (layer F.Cu) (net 9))
 (segment (start 133.35 92.71) (end 137.23319 92.71) (width 0.25) (layer F.Cu) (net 9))
 (segment (start 143.9 90.805) (end 143.9 88.655) (width 0.25) (layer F.Cu) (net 9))
 (segment (start 143.58319 88.33819) (end 141.605 88.33819) (width 0.25) (layer F.Cu) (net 9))
 (segment (start 143.9 88.655) (end 143.58319 88.33819) (width 0.25) (layer F.Cu) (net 9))
 (segment (start 137.23319 92.71) (end 141.605 88.33819) (width 0.25) (layer F.Cu) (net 9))
 (segment (start 160.655 103.105) (end 160.655 103.505) (width 0.25) (layer F.Cu) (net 9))
 (segment (start 157.88 100.33) (end 160.655 103.105) (width 0.25) (layer F.Cu) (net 9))
 (segment (start 153.67 100.33) (end 157.88 100.33) (width 0.25) (layer F.Cu) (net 9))
 (segment (start 142.24 92.71) (end 144.145 94.615) (width 0.25) (layer F.Cu) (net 9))
 (segment (start 144.145 94.615) (end 150.495 94.615) (width 0.25) (layer F.Cu) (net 9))
 (segment (start 150.495 94.615) (end 151.13 95.25) (width 0.25) (layer F.Cu) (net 9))
 (segment (start 137.23319 92.71) (end 142.24 92.71) (width 0.25) (layer F.Cu) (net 9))
 (segment (start 151.13 95.25) (end 151.13 97.79) (width 0.25) (layer F.Cu) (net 9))
 (segment (start 151.13 97.79) (end 153.67 100.33) (width 0.25) (layer F.Cu) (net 9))
 (segment (start 150.25 83.514682) (end 147.749451 81.014133) (width 0.25) (layer F.Cu) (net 10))
 (segment (start 150.25 90.805) (end 150.25 83.514682) (width 0.25) (layer F.Cu) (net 10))
 (segment (start 150.25 90.805) (end 152.4 90.805) (width 0.25) (layer F.Cu) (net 10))
 (via (at 154.305 92.62) (size 0.8) (drill 0.4) (layers F.Cu B.Cu) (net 10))
 (segment (start 152.4 90.805) (end 154.215 92.62) (width 0.25) (layer F.Cu) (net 10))
 (segment (start 154.215 92.62) (end 154.305 92.62) (width 0.25) (layer F.Cu) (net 10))
 (via (at 159.385 93.98) (size 0.8) (drill 0.4) (layers F.Cu B.Cu) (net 10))
 (segment (start 154.305 92.62) (end 158.025 92.62) (width 0.25) (layer B.Cu) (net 10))
 (segment (start 158.025 92.62) (end 159.385 93.98) (width 0.25) (layer B.Cu) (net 10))
 (via (at 165.1 93.98) (size 0.8) (drill 0.4) (layers F.Cu B.Cu) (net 10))
 (segment (start 159.385 93.98) (end 165.1 93.98) (width 0.25) (layer F.Cu) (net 10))
 (via (at 171.54 93.98) (size 0.8) (drill 0.4) (layers F.Cu B.Cu) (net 10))
 (segment (start 165.1 93.98) (end 171.54 93.98) (width 0.25) (layer B.Cu) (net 10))
 (via (at 173.445 92.71) (size 0.8) (drill 0.4) (layers F.Cu B.Cu) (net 10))
 (segment (start 171.54 93.98) (end 172.175 93.98) (width 0.25) (layer F.Cu) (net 10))
 (segment (start 172.175 93.98) (end 173.445 92.71) (width 0.25) (layer F.Cu) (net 10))
 (via (at 173.315 102.87) (size 0.8) (drill 0.4) (layers F.Cu B.Cu) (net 10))
 (segment (start 173.445 92.71) (end 173.445 102.74) (width 0.25) (layer B.Cu) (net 10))
 (segment (start 173.445 102.74) (end 173.315 102.87) (width 0.25) (layer B.Cu) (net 10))
 (segment (start 170.14 99.695) (end 173.315 102.87) (width 0.25) (layer F.Cu) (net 10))
 (segment (start 166.605 99.695) (end 170.14 99.695) (width 0.25) (layer F.Cu) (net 10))
 (segment (start 164.7 101.6) (end 166.605 99.695) (width 0.25) (layer F.Cu) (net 10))
 (segment (start 163.195 101.6) (end 164.7 101.6) (width 0.25) (layer F.Cu) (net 10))
 (segment (start 163.195 103.505) (end 163.195 101.6) (width 0.25) (layer F.Cu) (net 10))
 (segment (start 156.6 90.805) (end 156.6 87.24) (width 0.25) (layer F.Cu) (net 11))
 (segment (start 156.6 87.24) (end 158.115 85.725) (width 0.25) (layer F.Cu) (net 11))
 (segment (start 163.098584 85.725) (end 165.269451 83.554133) (width 0.25) (layer F.Cu) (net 11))
 (segment (start 158.115 85.725) (end 163.098584 85.725) (width 0.25) (layer F.Cu) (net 11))
 (segment (start 154.55 90.805) (end 154.55 89.145) (width 0.25) (layer F.Cu) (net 12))
 (segment (start 154.55 89.145) (end 153.035 87.63) (width 0.25) (layer F.Cu) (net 12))
 (segment (start 153.035 87.63) (end 153.035 81.28) (width 0.25) (layer F.Cu) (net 12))
 (segment (start 153.300867 81.014133) (end 155.109451 81.014133) (width 0.25) (layer F.Cu) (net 12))
 (segment (start 153.035 81.28) (end 153.300867 81.014133) (width 0.25) (layer F.Cu) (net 12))
 (segment (start 163.595 90.805) (end 162.95 90.805) (width 0.25) (layer F.Cu) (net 13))
 (segment (start 168.275 95.485) (end 163.595 90.805) (width 0.25) (layer F.Cu) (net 13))
 (segment (start 168.275 95.885) (end 168.275 95.485) (width 0.25) (layer F.Cu) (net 13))
 (segment (start 162.95 90.805) (end 162.95 89.78) (width 0.25) (layer F.Cu) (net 13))
 (via (at 163.83 88.9) (size 0.8) (drill 0.4) (layers F.Cu B.Cu) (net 13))
 (segment (start 162.95 89.78) (end 163.83 88.9) (width 0.25) (layer F.Cu) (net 13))
 (via (at 161.29 80.645) (size 0.8) (drill 0.4) (layers F.Cu B.Cu) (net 13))
 (segment (start 163.83 88.9) (end 161.29 86.36) (width 0.25) (layer B.Cu) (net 13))
 (segment (start 161.29 86.36) (end 161.29 80.645) (width 0.25) (layer B.Cu) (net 13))
 (segment (start 161.29 80.645) (end 160.02 80.645) (width 0.25) (layer F.Cu) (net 13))
 (segment (start 159.650867 81.014133) (end 157.909451 81.014133) (width 0.25) (layer F.Cu) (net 13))
 (segment (start 160.02 80.645) (end 159.650867 81.014133) (width 0.25) (layer F.Cu) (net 13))
 (segment (start 170.815 92.32) (end 169.3 90.805) (width 0.25) (layer F.Cu) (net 14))
 (segment (start 168.069451 81.014133) (end 169.279133 81.014133) (width 0.25) (layer F.Cu) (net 14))
 (segment (start 169.279133 81.014133) (end 169.545 81.28) (width 0.25) (layer F.Cu) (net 14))
 (segment (start 169.545 81.28) (end 169.545 85.725) (width 0.25) (layer F.Cu) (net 14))
 (via (at 167.005 88.265) (size 0.8) (drill 0.4) (layers F.Cu B.Cu) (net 14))
 (segment (start 169.545 85.725) (end 167.005 88.265) (width 0.25) (layer F.Cu) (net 14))
 (segment (start 167.005 88.265) (end 167.005 92.71) (width 0.25) (layer B.Cu) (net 14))
 (via (at 167.005 92.71) (size 0.8) (drill 0.4) (layers F.Cu B.Cu) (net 14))
 (segment (start 167.005 92.71) (end 170.815 92.71) (width 0.25) (layer F.Cu) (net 14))
 (segment (start 170.815 95.885) (end 170.815 92.71) (width 0.25) (layer F.Cu) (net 14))
 (segment (start 170.815 92.71) (end 170.815 92.32) (width 0.25) (layer F.Cu) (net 14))
 (segment (start 173.6 90.805) (end 173.6 89.29) (width 0.25) (layer F.Cu) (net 15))
 (via (at 178.435 87.63) (size 0.8) (drill 0.4) (layers F.Cu B.Cu) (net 15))
 (segment (start 173.6 89.29) (end 175.26 87.63) (width 0.25) (layer F.Cu) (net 15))
 (segment (start 175.26 87.63) (end 178.435 87.63) (width 0.25) (layer F.Cu) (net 15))
 (via (at 172.085 80.01) (size 0.8) (drill 0.4) (layers F.Cu B.Cu) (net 15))
 (segment (start 174.528584 81.915) (end 175.429451 81.014133) (width 0.25) (layer F.Cu) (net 15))
 (segment (start 172.085 80.01) (end 172.085 81.915) (width 0.25) (layer F.Cu) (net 15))
 (segment (start 172.085 81.915) (end 174.528584 81.915) (width 0.25) (layer F.Cu) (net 15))
 (segment (start 173.355 78.74) (end 172.085 80.01) (width 0.25) (layer B.Cu) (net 15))
 (segment (start 179.705 78.74) (end 173.355 78.74) (width 0.25) (layer B.Cu) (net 15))
 (segment (start 182.88 81.915) (end 179.705 78.74) (width 0.25) (layer B.Cu) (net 15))
 (segment (start 182.88 86.36) (end 182.88 81.915) (width 0.25) (layer B.Cu) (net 15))
 (segment (start 178.435 87.63) (end 181.61 87.63) (width 0.25) (layer B.Cu) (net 15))
 (segment (start 181.61 87.63) (end 182.88 86.36) (width 0.25) (layer B.Cu) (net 15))
 (via (at 178.435 90.805) (size 0.8) (drill 0.4) (layers F.Cu B.Cu) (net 16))
 (segment (start 175.65 90.805) (end 178.435 90.805) (width 0.25) (layer F.Cu) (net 16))
 (via (at 185.42 86.36) (size 0.8) (drill 0.4) (layers F.Cu B.Cu) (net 16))
 (segment (start 178.435 90.805) (end 180.975 90.805) (width 0.25) (layer B.Cu) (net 16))
 (segment (start 180.975 90.805) (end 185.42 86.36) (width 0.25) (layer B.Cu) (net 16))
 (segment (start 187.325 85.289682) (end 185.589451 83.554133) (width 0.25) (layer F.Cu) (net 16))
 (segment (start 187.325 85.725) (end 187.325 85.289682) (width 0.25) (layer F.Cu) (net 16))
 (segment (start 185.42 86.36) (end 186.69 86.36) (width 0.25) (layer F.Cu) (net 16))
 (segment (start 186.69 86.36) (end 187.325 85.725) (width 0.25) (layer F.Cu) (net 16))
 (segment (start 178.229451 81.014133) (end 182 84.784682) (width 0.25) (layer F.Cu) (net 17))
 (via (at 180.34 86.36) (size 0.8) (drill 0.4) (layers F.Cu B.Cu) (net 17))
 (segment (start 181.61 85.09) (end 182 85.09) (width 0.25) (layer F.Cu) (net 17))
 (segment (start 180.34 86.36) (end 181.61 85.09) (width 0.25) (layer F.Cu) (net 17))
 (segment (start 182 84.784682) (end 182 85.09) (width 0.25) (layer F.Cu) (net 17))
 (segment (start 182 85.09) (end 182 90.805) (width 0.25) (layer F.Cu) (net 17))
 (segment (start 165.1 86.36) (end 180.34 86.36) (width 0.25) (layer B.Cu) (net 17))
 (segment (start 165.1 88.9) (end 165.1 86.36) (width 0.25) (layer B.Cu) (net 17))
 (segment (start 160.655 95.885) (end 160.655 93.345) (width 0.25) (layer B.Cu) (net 17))
 (segment (start 160.655 93.345) (end 165.1 88.9) (width 0.25) (layer B.Cu) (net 17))
 (segment (start 189.865 82.489682) (end 188.389451 81.014133) (width 0.25) (layer F.Cu) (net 18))
 (segment (start 189.865 87.63) (end 189.865 82.489682) (width 0.25) (layer F.Cu) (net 18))
 (segment (start 188.35 90.805) (end 188.35 89.145) (width 0.25) (layer F.Cu) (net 18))
 (segment (start 188.35 89.145) (end 189.865 87.63) (width 0.25) (layer F.Cu) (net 18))
 (segment (start 165.735 96.285) (end 165.735 95.885) (width 0.25) (layer F.Cu) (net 18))
 (segment (start 167.24 97.79) (end 165.735 96.285) (width 0.25) (layer F.Cu) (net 18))
 (segment (start 185.81 93.345) (end 173.99 93.345) (width 0.25) (layer F.Cu) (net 18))
 (segment (start 188.35 90.805) (end 185.81 93.345) (width 0.25) (layer F.Cu) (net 18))
 (segment (start 173.99 93.345) (end 173.355 93.98) (width 0.25) (layer F.Cu) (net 18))
 (segment (start 173.355 93.98) (end 173.355 96.52) (width 0.25) (layer F.Cu) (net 18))
 (segment (start 173.355 96.52) (end 172.085 97.79) (width 0.25) (layer F.Cu) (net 18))
 (segment (start 172.085 97.79) (end 167.24 97.79) (width 0.25) (layer F.Cu) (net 18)))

